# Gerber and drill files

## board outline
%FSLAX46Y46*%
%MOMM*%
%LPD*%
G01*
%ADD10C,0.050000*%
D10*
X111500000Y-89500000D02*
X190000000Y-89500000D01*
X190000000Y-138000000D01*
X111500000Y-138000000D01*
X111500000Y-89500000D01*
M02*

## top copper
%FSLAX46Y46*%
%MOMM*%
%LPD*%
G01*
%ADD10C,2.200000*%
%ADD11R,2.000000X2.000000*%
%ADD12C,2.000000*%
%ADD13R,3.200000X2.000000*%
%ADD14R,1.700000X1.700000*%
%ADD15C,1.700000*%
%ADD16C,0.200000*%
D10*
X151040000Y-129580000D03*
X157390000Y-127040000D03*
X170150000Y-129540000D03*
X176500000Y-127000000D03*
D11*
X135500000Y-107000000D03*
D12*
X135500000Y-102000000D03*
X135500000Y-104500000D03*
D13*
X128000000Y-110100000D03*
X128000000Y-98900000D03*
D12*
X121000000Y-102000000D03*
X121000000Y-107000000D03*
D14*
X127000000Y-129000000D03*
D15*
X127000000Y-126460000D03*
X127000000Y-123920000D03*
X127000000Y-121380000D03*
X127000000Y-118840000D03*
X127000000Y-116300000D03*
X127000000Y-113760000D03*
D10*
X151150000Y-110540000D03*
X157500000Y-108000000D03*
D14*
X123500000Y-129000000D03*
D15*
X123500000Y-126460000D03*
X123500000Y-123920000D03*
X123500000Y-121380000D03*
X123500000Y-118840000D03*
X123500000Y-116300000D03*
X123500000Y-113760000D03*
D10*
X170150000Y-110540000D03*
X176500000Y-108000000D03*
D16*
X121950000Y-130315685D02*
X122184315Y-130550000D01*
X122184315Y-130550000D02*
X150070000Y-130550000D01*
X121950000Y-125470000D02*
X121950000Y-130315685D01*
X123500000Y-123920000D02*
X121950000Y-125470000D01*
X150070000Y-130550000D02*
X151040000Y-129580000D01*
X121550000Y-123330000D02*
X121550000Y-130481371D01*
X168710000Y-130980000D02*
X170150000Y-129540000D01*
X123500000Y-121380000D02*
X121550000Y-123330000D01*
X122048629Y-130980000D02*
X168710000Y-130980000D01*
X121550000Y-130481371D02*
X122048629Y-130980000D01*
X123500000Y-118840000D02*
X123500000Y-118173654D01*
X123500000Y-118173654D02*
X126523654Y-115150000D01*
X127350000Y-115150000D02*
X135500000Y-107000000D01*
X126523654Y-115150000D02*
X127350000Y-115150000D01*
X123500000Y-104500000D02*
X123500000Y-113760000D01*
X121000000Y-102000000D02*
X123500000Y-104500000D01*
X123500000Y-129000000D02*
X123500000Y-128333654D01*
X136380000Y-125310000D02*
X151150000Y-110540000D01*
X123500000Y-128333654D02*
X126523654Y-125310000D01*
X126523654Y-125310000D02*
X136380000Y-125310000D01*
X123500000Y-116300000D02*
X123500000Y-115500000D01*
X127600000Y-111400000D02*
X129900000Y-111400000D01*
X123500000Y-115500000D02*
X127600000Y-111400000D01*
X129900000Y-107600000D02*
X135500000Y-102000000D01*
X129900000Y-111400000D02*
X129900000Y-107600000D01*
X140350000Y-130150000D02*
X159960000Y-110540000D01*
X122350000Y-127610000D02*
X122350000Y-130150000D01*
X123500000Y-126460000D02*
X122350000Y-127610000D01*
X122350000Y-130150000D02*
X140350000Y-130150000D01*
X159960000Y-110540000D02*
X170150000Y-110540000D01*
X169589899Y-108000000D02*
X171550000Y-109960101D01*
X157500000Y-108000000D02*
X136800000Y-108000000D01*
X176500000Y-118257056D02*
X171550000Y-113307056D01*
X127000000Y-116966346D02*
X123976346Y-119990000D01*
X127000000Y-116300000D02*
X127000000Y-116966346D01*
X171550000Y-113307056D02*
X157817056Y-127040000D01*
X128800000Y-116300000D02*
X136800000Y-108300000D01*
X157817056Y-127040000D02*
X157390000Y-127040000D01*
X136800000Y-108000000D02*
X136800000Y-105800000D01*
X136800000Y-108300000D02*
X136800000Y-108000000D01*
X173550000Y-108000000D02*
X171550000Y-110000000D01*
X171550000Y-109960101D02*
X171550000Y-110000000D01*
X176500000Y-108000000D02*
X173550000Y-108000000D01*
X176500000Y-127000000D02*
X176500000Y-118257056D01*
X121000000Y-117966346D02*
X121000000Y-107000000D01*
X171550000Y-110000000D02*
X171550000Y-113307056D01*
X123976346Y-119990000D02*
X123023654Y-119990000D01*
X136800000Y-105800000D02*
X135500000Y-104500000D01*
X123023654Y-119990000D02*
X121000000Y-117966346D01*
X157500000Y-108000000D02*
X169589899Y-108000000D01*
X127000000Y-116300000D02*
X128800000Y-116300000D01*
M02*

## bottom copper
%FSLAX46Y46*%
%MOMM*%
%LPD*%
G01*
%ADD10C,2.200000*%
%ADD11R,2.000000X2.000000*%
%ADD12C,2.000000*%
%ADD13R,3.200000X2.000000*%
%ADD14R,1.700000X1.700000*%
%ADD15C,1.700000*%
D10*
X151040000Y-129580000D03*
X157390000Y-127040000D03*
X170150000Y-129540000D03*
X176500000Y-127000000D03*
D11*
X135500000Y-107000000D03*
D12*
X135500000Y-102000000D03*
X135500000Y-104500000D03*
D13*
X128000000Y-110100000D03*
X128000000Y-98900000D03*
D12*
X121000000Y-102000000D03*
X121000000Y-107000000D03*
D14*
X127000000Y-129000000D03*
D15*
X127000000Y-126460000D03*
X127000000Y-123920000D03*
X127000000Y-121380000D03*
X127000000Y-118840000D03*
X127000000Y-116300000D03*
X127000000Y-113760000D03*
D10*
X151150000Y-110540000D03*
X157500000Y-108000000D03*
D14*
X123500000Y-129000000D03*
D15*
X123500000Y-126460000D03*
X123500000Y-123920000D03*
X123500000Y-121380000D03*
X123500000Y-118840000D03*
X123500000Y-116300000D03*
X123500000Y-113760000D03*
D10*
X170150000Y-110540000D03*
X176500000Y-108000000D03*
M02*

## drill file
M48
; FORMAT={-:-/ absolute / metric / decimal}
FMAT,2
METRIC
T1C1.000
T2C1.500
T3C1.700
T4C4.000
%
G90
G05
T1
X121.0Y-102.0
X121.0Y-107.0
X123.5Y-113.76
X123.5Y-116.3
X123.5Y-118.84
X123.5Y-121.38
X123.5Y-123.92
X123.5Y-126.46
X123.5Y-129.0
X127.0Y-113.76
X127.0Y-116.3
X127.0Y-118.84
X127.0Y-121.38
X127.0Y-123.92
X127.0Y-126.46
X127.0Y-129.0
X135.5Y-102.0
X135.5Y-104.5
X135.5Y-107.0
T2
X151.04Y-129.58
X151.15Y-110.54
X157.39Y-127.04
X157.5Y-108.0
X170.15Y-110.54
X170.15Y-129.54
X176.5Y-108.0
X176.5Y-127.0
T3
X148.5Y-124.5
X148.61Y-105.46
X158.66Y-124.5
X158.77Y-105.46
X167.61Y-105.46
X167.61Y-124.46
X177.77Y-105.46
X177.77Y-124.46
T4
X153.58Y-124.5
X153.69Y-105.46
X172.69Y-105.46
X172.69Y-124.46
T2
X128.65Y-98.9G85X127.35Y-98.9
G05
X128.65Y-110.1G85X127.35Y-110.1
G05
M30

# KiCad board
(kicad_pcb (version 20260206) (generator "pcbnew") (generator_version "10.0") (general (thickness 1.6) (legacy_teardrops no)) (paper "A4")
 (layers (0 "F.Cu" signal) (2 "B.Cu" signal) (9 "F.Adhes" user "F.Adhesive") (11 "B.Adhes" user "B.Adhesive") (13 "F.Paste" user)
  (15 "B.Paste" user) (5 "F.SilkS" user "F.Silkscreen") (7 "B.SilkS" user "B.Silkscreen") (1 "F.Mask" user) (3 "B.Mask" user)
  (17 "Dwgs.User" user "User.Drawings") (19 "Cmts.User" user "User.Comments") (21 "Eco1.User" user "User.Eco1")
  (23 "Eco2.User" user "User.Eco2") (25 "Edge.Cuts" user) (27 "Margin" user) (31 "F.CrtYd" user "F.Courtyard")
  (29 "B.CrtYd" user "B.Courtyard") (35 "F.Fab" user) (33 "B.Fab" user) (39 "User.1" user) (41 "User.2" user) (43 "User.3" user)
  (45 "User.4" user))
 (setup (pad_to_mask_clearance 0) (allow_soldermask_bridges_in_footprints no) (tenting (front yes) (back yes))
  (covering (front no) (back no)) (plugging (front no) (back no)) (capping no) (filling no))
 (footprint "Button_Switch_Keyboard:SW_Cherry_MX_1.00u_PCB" (layer "F.Cu") (at 151.04 129.58 180)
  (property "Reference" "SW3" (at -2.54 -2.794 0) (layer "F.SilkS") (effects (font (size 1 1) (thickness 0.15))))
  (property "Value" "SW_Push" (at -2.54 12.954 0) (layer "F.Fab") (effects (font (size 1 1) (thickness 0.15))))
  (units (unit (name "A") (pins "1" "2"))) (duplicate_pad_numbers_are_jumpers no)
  (pad "" np_thru_hole circle (at -7.62 5.08 180) (size 1.7 1.7) (drill 1.7) (layers "*.Cu" "*.Mask"))
  (pad "" np_thru_hole circle (at -2.54 5.08 180) (size 4 4) (drill 4) (layers "*.Cu" "*.Mask"))
  (pad "" np_thru_hole circle (at 2.54 5.08 180) (size 1.7 1.7) (drill 1.7) (layers "*.Cu" "*.Mask"))
  (pad "1" thru_hole circle (at 0 0 180) (size 2.2 2.2) (drill 1.5) (layers "*.Cu" "*.Mask") (remove_unused_layers no)
   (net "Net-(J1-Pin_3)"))
  (pad "2" thru_hole circle (at -6.35 2.54 180) (size 2.2 2.2) (drill 1.5) (layers "*.Cu" "*.Mask") (remove_unused_layers no) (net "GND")))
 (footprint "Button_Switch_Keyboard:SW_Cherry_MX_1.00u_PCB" (layer "F.Cu") (at 170.15 129.54 180)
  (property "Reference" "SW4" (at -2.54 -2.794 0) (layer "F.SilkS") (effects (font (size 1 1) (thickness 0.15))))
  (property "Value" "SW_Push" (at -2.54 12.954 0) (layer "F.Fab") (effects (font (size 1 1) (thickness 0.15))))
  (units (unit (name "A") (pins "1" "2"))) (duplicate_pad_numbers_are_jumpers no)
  (pad "" np_thru_hole circle (at -7.62 5.08 180) (size 1.7 1.7) (drill 1.7) (layers "*.Cu" "*.Mask"))
  (pad "" np_thru_hole circle (at -2.54 5.08 180) (size 4 4) (drill 4) (layers "*.Cu" "*.Mask"))
  (pad "" np_thru_hole circle (at 2.54 5.08 180) (size 1.7 1.7) (drill 1.7) (layers "*.Cu" "*.Mask"))
  (pad "1" thru_hole circle (at 0 0 180) (size 2.2 2.2) (drill 1.5) (layers "*.Cu" "*.Mask") (remove_unused_layers no)
   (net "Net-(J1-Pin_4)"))
  (pad "2" thru_hole circle (at -6.35 2.54 180) (size 2.2 2.2) (drill 1.5) (layers "*.Cu" "*.Mask") (remove_unused_layers no) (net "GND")))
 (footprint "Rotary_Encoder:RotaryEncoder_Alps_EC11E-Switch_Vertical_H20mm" (layer "F.Cu") (at 135.5 107 180)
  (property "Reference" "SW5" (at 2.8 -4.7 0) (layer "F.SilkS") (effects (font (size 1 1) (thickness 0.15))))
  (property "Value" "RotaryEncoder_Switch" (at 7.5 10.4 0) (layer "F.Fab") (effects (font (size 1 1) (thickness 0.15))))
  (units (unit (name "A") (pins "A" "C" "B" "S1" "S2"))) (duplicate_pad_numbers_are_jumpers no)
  (pad "A" thru_hole rect (at 0 0 180) (size 2 2) (drill 1) (layers "*.Cu" "*.Mask") (remove_unused_layers no) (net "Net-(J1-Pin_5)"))
  (pad "B" thru_hole circle (at 0 5 180) (size 2 2) (drill 1) (layers "*.Cu" "*.Mask") (remove_unused_layers no) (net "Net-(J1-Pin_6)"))
  (pad "C" thru_hole circle (at 0 2.5 180) (size 2 2) (drill 1) (layers "*.Cu" "*.Mask") (remove_unused_layers no) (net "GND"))
  (pad "MP" thru_hole rect (at 7.5 -3.1 180) (size 3.2 2) (drill oval 2.8 1.5) (layers "*.Cu" "*.Mask") (remove_unused_layers no))
  (pad "MP" thru_hole rect (at 7.5 8.1 180) (size 3.2 2) (drill oval 2.8 1.5) (layers "*.Cu" "*.Mask") (remove_unused_layers no))
  (pad "S1" thru_hole circle (at 14.5 5 180) (size 2 2) (drill 1) (layers "*.Cu" "*.Mask") (remove_unused_layers no) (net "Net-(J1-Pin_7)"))
  (pad "S2" thru_hole circle (at 14.5 0 180) (size 2 2) (drill 1) (layers "*.Cu" "*.Mask") (remove_unused_layers no) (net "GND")))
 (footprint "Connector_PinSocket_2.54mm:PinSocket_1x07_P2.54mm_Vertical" (layer "F.Cu") (at 127 129 180)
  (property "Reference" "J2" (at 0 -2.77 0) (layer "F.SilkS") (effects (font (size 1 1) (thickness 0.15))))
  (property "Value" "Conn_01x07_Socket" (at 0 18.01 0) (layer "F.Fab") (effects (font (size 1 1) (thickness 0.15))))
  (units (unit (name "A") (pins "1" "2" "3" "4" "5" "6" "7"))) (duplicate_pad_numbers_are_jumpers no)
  (pad "1" thru_hole rect (at 0 0 180) (size 1.7 1.7) (drill 1) (layers "*.Cu" "*.Mask") (remove_unused_layers no)
   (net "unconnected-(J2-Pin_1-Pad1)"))
  (pad "2" thru_hole circle (at 0 2.54 180) (size 1.7 1.7) (drill 1) (layers "*.Cu" "*.Mask") (remove_unused_layers no)
   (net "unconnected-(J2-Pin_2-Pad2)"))
  (pad "3" thru_hole circle (at 0 5.08 180) (size 1.7 1.7) (drill 1) (layers "*.Cu" "*.Mask") (remove_unused_layers no)
   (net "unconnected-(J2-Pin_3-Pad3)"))
  (pad "4" thru_hole circle (at 0 7.62 180) (size 1.7 1.7) (drill 1) (layers "*.Cu" "*.Mask") (remove_unused_layers no)
   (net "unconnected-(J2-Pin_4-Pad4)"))
  (pad "5" thru_hole circle (at 0 10.16 180) (size 1.7 1.7) (drill 1) (layers "*.Cu" "*.Mask") (remove_unused_layers no)
   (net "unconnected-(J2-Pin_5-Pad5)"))
  (pad "6" thru_hole circle (at 0 12.7 180) (size 1.7 1.7) (drill 1) (layers "*.Cu" "*.Mask") (remove_unused_layers no) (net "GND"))
  (pad "7" thru_hole circle (at 0 15.24 180) (size 1.7 1.7) (drill 1) (layers "*.Cu" "*.Mask") (remove_unused_layers no)
   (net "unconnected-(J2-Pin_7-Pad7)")))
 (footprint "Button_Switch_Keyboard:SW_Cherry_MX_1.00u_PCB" (layer "F.Cu") (at 151.15 110.54 180)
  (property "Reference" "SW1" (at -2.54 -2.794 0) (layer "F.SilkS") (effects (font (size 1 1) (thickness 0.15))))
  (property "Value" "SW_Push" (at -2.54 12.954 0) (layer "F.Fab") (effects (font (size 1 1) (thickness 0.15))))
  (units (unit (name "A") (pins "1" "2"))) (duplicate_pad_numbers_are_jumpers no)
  (pad "" np_thru_hole circle (at -7.62 5.08 180) (size 1.7 1.7) (drill 1.7) (layers "*.Cu" "*.Mask"))
  (pad "" np_thru_hole circle (at -2.54 5.08 180) (size 4 4) (drill 4) (layers "*.Cu" "*.Mask"))
  (pad "" np_thru_hole circle (at 2.54 5.08 180) (size 1.7 1.7) (drill 1.7) (layers "*.Cu" "*.Mask"))
  (pad "1" thru_hole circle (at 0 0 180) (size 2.2 2.2) (drill 1.5) (layers "*.Cu" "*.Mask") (remove_unused_layers no)
   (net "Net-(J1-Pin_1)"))
  (pad "2" thru_hole circle (at -6.35 2.54 180) (size 2.2 2.2) (drill 1.5) (layers "*.Cu" "*.Mask") (remove_unused_layers no) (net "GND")))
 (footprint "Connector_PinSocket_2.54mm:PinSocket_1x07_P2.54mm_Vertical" (layer "F.Cu") (at 123.5 129 180)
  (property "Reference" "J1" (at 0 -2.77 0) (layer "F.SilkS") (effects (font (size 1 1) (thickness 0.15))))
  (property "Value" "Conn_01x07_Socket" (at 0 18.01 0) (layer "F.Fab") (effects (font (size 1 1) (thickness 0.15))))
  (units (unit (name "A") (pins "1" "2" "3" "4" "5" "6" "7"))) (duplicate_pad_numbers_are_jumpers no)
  (pad "1" thru_hole rect (at 0 0 180) (size 1.7 1.7) (drill 1) (layers "*.Cu" "*.Mask") (remove_unused_layers no) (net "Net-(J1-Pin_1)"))
  (pad "2" thru_hole circle (at 0 2.54 180) (size 1.7 1.7) (drill 1) (layers "*.Cu" "*.Mask") (remove_unused_layers no)
   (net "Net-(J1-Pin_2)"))
  (pad "3" thru_hole circle (at 0 5.08 180) (size 1.7 1.7) (drill 1) (layers "*.Cu" "*.Mask") (remove_unused_layers no)
   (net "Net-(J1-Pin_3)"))
  (pad "4" thru_hole circle (at 0 7.62 180) (size 1.7 1.7) (drill 1) (layers "*.Cu" "*.Mask") (remove_unused_layers no)
   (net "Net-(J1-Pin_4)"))
  (pad "5" thru_hole circle (at 0 10.16 180) (size 1.7 1.7) (drill 1) (layers "*.Cu" "*.Mask") (remove_unused_layers no)
   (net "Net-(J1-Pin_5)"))
  (pad "6" thru_hole circle (at 0 12.7 180) (size 1.7 1.7) (drill 1) (layers "*.Cu" "*.Mask") (remove_unused_layers no)
   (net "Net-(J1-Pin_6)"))
  (pad "7" thru_hole circle (at 0 15.24 180) (size 1.7 1.7) (drill 1) (layers "*.Cu" "*.Mask") (remove_unused_layers no)
   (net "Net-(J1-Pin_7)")))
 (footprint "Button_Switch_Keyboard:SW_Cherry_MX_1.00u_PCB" (layer "F.Cu") (at 170.15 110.54 180)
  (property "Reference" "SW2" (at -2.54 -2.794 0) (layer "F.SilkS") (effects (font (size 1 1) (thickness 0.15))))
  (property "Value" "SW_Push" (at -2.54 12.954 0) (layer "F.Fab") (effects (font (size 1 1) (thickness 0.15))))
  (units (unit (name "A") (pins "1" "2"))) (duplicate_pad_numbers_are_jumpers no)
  (pad "" np_thru_hole circle (at -7.62 5.08 180) (size 1.7 1.7) (drill 1.7) (layers "*.Cu" "*.Mask"))
  (pad "" np_thru_hole circle (at -2.54 5.08 180) (size 4 4) (drill 4) (layers "*.Cu" "*.Mask"))
  (pad "" np_thru_hole circle (at 2.54 5.08 180) (size 1.7 1.7) (drill 1.7) (layers "*.Cu" "*.Mask"))
  (pad "1" thru_hole circle (at 0 0 180) (size 2.2 2.2) (drill 1.5) (layers "*.Cu" "*.Mask") (remove_unused_layers no)
   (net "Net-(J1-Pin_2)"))
  (pad "2" thru_hole circle (at -6.35 2.54 180) (size 2.2 2.2) (drill 1.5) (layers "*.Cu" "*.Mask") (remove_unused_layers no) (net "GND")))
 (gr_rect (start 111.5 89.5) (end 190 138) (stroke (width 0.05) (type default)) (fill no) (layer "Edge.Cuts"))
 (segment (start 121.95 130.315685) (end 122.184315 130.55) (width 0.2) (layer "F.Cu") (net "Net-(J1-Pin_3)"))
 (segment (start 122.184315 130.55) (end 150.07 130.55) (width 0.2) (layer "F.Cu") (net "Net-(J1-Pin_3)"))
 (segment (start 121.95 125.47) (end 121.95 130.315685) (width 0.2) (layer "F.Cu") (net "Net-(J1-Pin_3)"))
 (segment (start 123.5 123.92) (end 121.95 125.47) (width 0.2) (layer "F.Cu") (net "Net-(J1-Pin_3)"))
 (segment (start 150.07 130.55) (end 151.04 129.58) (width 0.2) (layer "F.Cu") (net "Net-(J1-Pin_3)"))
 (segment (start 121.55 123.33) (end 121.55 130.481371) (width 0.2) (layer "F.Cu") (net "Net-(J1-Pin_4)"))
 (segment (start 168.71 130.98) (end 170.15 129.54) (width 0.2) (layer "F.Cu") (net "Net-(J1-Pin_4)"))
 (segment (start 123.5 121.38) (end 121.55 123.33) (width 0.2) (layer "F.Cu") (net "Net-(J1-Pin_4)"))
 (segment (start 122.048629 130.98) (end 168.71 130.98) (width 0.2) (layer "F.Cu") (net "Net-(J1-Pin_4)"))
 (segment (start 121.55 130.481371) (end 122.048629 130.98) (width 0.2) (layer "F.Cu") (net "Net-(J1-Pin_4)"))
 (segment (start 123.5 118.84) (end 123.5 118.173654) (width 0.2) (layer "F.Cu") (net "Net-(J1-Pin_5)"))
 (segment (start 123.5 118.173654) (end 126.523654 115.15) (width 0.2) (layer "F.Cu") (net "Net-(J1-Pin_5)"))
 (segment (start 127.35 115.15) (end 135.5 107) (width 0.2) (layer "F.Cu") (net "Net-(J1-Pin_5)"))
 (segment (start 126.523654 115.15) (end 127.35 115.15) (width 0.2) (layer "F.Cu") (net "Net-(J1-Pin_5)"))
 (segment (start 123.5 104.5) (end 123.5 113.76) (width 0.2) (layer "F.Cu") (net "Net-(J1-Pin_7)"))
 (segment (start 121 102) (end 123.5 104.5) (width 0.2) (layer "F.Cu") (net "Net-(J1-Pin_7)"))
 (segment (start 123.5 129) (end 123.5 128.333654) (width 0.2) (layer "F.Cu") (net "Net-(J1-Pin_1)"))
 (segment (start 136.38 125.31) (end 151.15 110.54) (width 0.2) (layer "F.Cu") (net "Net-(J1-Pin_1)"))
 (segment (start 123.5 128.333654) (end 126.523654 125.31) (width 0.2) (layer "F.Cu") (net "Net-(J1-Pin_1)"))
 (segment (start 126.523654 125.31) (end 136.38 125.31) (width 0.2) (layer "F.Cu") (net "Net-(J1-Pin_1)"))
 (segment (start 123.5 116.3) (end 123.5 115.5) (width 0.2) (layer "F.Cu") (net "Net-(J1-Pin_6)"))
 (segment (start 127.6 111.4) (end 129.9 111.4) (width 0.2) (layer "F.Cu") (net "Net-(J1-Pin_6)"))
 (segment (start 123.5 115.5) (end 127.6 111.4) (width 0.2) (layer "F.Cu") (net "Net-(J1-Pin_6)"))
 (segment (start 129.9 107.6) (end 135.5 102) (width 0.2) (layer "F.Cu") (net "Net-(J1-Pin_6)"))
 (segment (start 129.9 111.4) (end 129.9 107.6) (width 0.2) (layer "F.Cu") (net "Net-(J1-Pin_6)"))
 (segment (start 140.35 130.15) (end 159.96 110.54) (width 0.2) (layer "F.Cu") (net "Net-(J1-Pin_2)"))
 (segment (start 122.35 127.61) (end 122.35 130.15) (width 0.2) (layer "F.Cu") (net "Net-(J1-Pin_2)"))
 (segment (start 123.5 126.46) (end 122.35 127.61) (width 0.2) (layer "F.Cu") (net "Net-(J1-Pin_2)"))
 (segment (start 122.35 130.15) (end 140.35 130.15) (width 0.2) (layer "F.Cu") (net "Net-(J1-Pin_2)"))
 (segment (start 159.96 110.54) (end 170.15 110.54) (width 0.2) (layer "F.Cu") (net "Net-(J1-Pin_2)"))
 (segment (start 169.589899 108) (end 171.55 109.960101) (width 0.2) (layer "F.Cu") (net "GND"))
 (segment (start 157.5 108) (end 136.8 108) (width 0.2) (layer "F.Cu") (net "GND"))
 (segment (start 176.5 118.257056) (end 171.55 113.307056) (width 0.2) (layer "F.Cu") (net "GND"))
 (segment (start 127 116.966346) (end 123.976346 119.99) (width 0.2) (layer "F.Cu") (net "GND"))
 (segment (start 127 116.3) (end 127 116.966346) (width 0.2) (layer "F.Cu") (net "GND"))
 (segment (start 171.55 113.307056) (end 157.817056 127.04) (width 0.2) (layer "F.Cu") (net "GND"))
 (segment (start 128.8 116.3) (end 136.8 108.3) (width 0.2) (layer "F.Cu") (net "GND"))
 (segment (start 157.817056 127.04) (end 157.39 127.04) (width 0.2) (layer "F.Cu") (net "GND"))
 (segment (start 136.8 108) (end 136.8 105.8) (width 0.2) (layer "F.Cu") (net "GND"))
 (segment (start 136.8 108.3) (end 136.8 108) (width 0.2) (layer "F.Cu") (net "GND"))
 (segment (start 173.55 108) (end 171.55 110) (width 0.2) (layer "F.Cu") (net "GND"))
 (segment (start 171.55 109.960101) (end 171.55 110) (width 0.2) (layer "F.Cu") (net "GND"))
 (segment (start 176.5 108) (end 173.55 108) (width 0.2) (layer "F.Cu") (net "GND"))
 (segment (start 176.5 127) (end 176.5 118.257056) (width 0.2) (layer "F.Cu") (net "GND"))
 (segment (start 121 117.966346) (end 121 107) (width 0.2) (layer "F.Cu") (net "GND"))
 (segment (start 171.55 110) (end 171.55 113.307056) (width 0.2) (layer "F.Cu") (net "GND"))
 (segment (start 123.976346 119.99) (end 123.023654 119.99) (width 0.2) (layer "F.Cu") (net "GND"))
 (segment (start 136.8 105.8) (end 135.5 104.5) (width 0.2) (layer "F.Cu") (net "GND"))
 (segment (start 123.023654 119.99) (end 121 117.966346) (width 0.2) (layer "F.Cu") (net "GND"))
 (segment (start 157.5 108) (end 169.589899 108) (width 0.2) (layer "F.Cu") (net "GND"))
 (segment (start 127 116.3) (end 128.8 116.3) (width 0.2) (layer "F.Cu") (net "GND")))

